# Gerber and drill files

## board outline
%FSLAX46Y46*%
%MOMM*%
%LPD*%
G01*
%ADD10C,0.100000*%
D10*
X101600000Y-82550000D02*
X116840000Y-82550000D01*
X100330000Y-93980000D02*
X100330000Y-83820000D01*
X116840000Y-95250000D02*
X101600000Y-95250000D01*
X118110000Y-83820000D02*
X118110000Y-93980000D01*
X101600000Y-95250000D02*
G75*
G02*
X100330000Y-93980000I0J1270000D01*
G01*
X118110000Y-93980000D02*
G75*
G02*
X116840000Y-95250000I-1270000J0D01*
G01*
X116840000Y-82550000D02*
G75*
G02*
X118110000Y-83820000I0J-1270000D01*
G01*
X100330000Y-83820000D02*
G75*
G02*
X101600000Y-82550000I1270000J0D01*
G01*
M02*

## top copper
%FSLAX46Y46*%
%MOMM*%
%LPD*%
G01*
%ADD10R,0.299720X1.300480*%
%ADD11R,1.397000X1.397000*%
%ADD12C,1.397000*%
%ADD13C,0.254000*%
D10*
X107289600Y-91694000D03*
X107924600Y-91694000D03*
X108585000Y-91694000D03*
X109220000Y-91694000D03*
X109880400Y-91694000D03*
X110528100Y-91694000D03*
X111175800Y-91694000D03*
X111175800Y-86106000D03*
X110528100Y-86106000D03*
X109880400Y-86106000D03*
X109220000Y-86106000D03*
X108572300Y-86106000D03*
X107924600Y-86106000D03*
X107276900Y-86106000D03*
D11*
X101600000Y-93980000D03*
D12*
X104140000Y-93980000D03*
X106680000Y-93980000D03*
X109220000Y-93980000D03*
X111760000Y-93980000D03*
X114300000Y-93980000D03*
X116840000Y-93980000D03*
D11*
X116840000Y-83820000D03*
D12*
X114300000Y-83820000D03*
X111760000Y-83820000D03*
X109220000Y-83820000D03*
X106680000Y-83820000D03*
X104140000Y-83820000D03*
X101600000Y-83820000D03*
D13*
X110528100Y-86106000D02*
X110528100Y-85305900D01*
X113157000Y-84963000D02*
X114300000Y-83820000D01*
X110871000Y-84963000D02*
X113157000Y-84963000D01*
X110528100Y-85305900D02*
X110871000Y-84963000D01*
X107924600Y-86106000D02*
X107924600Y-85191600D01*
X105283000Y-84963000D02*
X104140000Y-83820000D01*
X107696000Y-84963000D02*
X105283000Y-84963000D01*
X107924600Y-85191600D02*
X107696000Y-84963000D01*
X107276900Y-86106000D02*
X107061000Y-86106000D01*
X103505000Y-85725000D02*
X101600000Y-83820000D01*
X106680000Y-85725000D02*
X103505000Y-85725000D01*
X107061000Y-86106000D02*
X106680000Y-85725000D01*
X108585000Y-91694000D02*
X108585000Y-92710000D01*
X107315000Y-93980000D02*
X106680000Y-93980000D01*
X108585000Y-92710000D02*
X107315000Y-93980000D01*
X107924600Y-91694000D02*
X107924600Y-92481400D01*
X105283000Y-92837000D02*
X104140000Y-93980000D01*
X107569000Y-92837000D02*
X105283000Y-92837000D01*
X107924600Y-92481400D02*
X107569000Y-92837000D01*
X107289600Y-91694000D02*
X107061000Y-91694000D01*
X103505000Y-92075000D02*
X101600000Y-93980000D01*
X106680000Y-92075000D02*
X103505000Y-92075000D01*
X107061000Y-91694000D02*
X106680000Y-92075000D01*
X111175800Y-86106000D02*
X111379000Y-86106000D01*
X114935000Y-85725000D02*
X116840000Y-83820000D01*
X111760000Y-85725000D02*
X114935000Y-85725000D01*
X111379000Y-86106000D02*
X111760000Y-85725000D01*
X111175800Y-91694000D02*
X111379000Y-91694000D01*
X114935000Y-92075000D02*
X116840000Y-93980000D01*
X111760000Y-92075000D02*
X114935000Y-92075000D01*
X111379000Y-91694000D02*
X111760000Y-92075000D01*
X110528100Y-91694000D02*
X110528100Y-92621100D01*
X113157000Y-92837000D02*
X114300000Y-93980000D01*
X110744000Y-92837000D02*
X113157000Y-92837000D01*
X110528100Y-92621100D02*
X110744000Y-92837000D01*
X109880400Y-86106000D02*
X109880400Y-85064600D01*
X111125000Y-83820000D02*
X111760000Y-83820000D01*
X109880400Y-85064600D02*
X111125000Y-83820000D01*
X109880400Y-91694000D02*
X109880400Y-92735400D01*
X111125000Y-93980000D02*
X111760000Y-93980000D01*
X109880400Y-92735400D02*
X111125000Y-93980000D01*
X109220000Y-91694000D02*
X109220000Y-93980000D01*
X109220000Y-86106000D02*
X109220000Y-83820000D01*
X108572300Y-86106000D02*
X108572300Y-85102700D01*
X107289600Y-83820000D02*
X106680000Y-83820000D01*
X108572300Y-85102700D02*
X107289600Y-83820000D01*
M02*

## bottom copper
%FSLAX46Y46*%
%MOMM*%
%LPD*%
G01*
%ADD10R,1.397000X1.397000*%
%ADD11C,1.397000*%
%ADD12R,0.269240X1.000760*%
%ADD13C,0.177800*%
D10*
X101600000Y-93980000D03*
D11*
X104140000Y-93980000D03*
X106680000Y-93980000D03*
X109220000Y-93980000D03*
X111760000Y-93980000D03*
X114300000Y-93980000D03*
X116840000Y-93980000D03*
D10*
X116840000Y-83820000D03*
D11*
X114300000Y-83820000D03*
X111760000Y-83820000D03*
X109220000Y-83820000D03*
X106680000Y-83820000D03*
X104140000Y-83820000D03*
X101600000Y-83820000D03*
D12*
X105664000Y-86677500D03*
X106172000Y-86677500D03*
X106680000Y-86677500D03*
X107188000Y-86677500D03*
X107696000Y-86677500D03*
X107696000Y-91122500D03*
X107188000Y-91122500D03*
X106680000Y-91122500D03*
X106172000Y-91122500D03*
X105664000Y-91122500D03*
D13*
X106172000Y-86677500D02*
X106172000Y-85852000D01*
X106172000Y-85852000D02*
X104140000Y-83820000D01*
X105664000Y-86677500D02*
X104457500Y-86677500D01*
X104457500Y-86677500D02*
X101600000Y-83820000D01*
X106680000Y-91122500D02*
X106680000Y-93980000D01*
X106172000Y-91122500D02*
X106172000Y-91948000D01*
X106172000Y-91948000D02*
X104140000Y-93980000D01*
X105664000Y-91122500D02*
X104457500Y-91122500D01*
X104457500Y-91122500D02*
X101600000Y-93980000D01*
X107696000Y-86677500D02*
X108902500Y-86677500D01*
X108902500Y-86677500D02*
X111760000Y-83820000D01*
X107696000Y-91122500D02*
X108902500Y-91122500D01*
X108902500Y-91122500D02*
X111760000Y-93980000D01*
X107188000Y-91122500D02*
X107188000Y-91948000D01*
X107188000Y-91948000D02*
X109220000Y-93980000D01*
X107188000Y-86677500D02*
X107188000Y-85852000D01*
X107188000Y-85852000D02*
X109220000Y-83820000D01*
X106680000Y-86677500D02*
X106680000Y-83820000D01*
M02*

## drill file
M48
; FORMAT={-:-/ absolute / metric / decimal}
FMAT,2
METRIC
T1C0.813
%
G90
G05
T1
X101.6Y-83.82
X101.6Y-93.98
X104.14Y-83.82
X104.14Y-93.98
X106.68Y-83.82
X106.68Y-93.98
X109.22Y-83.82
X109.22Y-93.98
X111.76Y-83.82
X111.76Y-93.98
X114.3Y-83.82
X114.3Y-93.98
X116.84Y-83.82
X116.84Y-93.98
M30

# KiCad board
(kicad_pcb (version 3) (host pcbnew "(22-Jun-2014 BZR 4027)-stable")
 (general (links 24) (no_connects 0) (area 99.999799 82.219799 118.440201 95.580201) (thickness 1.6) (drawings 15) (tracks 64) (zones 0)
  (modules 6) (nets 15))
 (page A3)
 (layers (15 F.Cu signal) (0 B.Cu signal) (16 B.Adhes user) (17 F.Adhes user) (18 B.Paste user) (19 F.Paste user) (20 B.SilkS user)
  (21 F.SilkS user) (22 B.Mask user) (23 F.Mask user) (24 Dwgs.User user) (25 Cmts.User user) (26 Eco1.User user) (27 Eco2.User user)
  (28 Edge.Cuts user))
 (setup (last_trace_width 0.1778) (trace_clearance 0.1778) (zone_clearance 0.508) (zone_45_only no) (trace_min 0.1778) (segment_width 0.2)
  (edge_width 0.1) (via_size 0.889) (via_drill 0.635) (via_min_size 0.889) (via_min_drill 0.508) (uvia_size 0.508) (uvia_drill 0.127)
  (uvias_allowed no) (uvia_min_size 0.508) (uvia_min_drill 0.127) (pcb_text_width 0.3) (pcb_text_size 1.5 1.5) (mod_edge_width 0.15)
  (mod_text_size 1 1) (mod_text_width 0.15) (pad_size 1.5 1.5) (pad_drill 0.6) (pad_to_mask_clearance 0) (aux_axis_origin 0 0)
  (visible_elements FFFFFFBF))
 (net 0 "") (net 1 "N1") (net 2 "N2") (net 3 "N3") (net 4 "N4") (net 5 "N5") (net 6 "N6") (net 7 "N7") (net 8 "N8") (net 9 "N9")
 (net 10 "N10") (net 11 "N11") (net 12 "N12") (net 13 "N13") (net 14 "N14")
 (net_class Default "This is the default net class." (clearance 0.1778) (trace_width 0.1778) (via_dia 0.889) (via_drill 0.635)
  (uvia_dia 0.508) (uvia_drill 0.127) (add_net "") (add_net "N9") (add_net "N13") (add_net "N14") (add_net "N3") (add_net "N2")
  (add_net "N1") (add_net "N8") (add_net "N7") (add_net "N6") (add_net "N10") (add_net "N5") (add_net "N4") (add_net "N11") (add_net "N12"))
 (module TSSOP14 (layer F.Cu) (at 109.22 88.9)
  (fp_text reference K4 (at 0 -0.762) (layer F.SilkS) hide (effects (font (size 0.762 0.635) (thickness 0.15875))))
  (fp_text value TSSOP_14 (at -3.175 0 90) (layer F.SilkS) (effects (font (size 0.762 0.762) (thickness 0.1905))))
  (pad 1 smd rect (at -1.9304 2.794) (size 0.29972 1.30048) (layers F.Cu F.Paste F.Mask) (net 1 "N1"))
  (pad 2 smd rect (at -1.2954 2.794) (size 0.29972 1.30048) (layers F.Cu F.Paste F.Mask) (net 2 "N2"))
  (pad 3 smd rect (at -0.635 2.794) (size 0.29972 1.30048) (layers F.Cu F.Paste F.Mask) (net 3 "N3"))
  (pad 4 smd rect (at 0 2.794) (size 0.29972 1.30048) (layers F.Cu F.Paste F.Mask) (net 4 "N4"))
  (pad 5 smd rect (at 0.6604 2.794) (size 0.29972 1.30048) (layers F.Cu F.Paste F.Mask) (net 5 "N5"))
  (pad 6 smd rect (at 1.3081 2.794) (size 0.29972 1.30048) (layers F.Cu F.Paste F.Mask) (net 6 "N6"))
  (pad 7 smd rect (at 1.9558 2.794) (size 0.29972 1.30048) (layers F.Cu F.Paste F.Mask) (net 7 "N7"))
  (pad 8 smd rect (at 1.9558 -2.794) (size 0.29972 1.30048) (layers F.Cu F.Paste F.Mask) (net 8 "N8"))
  (pad 9 smd rect (at 1.3081 -2.794) (size 0.29972 1.30048) (layers F.Cu F.Paste F.Mask) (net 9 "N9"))
  (pad 10 smd rect (at 0.6604 -2.794) (size 0.29972 1.30048) (layers F.Cu F.Paste F.Mask) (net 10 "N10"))
  (pad 11 smd rect (at 0 -2.794) (size 0.29972 1.30048) (layers F.Cu F.Paste F.Mask) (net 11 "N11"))
  (pad 12 smd rect (at -0.6477 -2.794) (size 0.29972 1.30048) (layers F.Cu F.Paste F.Mask) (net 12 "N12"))
  (pad 13 smd rect (at -1.2954 -2.794) (size 0.29972 1.30048) (layers F.Cu F.Paste F.Mask) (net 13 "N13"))
  (pad 14 smd rect (at -1.9431 -2.794) (size 0.29972 1.30048) (layers F.Cu F.Paste F.Mask) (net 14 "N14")))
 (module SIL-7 (layer F.Cu) (at 109.22 93.98)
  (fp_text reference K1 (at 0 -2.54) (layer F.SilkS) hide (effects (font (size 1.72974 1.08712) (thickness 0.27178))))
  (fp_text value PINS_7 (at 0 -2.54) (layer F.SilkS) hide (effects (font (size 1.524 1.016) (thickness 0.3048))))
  (pad 1 thru_hole rect (at -7.62 0) (size 1.397 1.397) (drill 0.8128) (layers *.Cu *.Mask F.SilkS) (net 1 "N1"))
  (pad 2 thru_hole circle (at -5.08 0) (size 1.397 1.397) (drill 0.8128) (layers *.Cu *.SilkS *.Mask) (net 2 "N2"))
  (pad 3 thru_hole circle (at -2.54 0) (size 1.397 1.397) (drill 0.8128) (layers *.Cu *.SilkS *.Mask) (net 3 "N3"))
  (pad 4 thru_hole circle (at 0 0) (size 1.397 1.397) (drill 0.8128) (layers *.Cu *.SilkS *.Mask) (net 4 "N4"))
  (pad 5 thru_hole circle (at 2.54 0) (size 1.397 1.397) (drill 0.8128) (layers *.Cu *.SilkS *.Mask) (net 5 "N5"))
  (pad 6 thru_hole circle (at 5.08 0) (size 1.397 1.397) (drill 0.8128) (layers *.Cu *.SilkS *.Mask) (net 6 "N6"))
  (pad 7 thru_hole circle (at 7.62 0) (size 1.397 1.397) (drill 0.8128) (layers *.Cu *.SilkS *.Mask) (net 7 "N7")))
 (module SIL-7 (layer F.Cu) (at 109.22 83.82 180)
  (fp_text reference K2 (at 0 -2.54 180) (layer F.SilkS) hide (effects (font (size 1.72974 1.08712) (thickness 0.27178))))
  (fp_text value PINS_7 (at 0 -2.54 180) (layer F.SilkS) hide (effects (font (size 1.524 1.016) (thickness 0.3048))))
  (pad 1 thru_hole rect (at -7.62 0 180) (size 1.397 1.397) (drill 0.8128) (layers *.Cu *.Mask F.SilkS) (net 8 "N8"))
  (pad 2 thru_hole circle (at -5.08 0 180) (size 1.397 1.397) (drill 0.8128) (layers *.Cu *.SilkS *.Mask) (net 9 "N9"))
  (pad 3 thru_hole circle (at -2.54 0 180) (size 1.397 1.397) (drill 0.8128) (layers *.Cu *.SilkS *.Mask) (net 10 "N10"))
  (pad 4 thru_hole circle (at 0 0 180) (size 1.397 1.397) (drill 0.8128) (layers *.Cu *.SilkS *.Mask) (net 11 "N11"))
  (pad 5 thru_hole circle (at 2.54 0 180) (size 1.397 1.397) (drill 0.8128) (layers *.Cu *.SilkS *.Mask) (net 12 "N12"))
  (pad 6 thru_hole circle (at 5.08 0 180) (size 1.397 1.397) (drill 0.8128) (layers *.Cu *.SilkS *.Mask) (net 13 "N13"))
  (pad 7 thru_hole circle (at 7.62 0 180) (size 1.397 1.397) (drill 0.8128) (layers *.Cu *.SilkS *.Mask) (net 14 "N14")))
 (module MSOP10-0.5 (layer B.Cu) (at 106.68 88.9)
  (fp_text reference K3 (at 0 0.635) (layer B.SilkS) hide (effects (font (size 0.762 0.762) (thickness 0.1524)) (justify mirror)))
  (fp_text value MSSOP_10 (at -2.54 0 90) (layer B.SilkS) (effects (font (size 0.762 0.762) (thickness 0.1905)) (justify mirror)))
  (pad 1 smd rect (at -1.016 -2.2225) (size 0.26924 1.00076) (layers B.Cu B.Paste B.Mask) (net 14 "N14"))
  (pad 2 smd rect (at -0.508 -2.2225) (size 0.26924 1.00076) (layers B.Cu B.Paste B.Mask) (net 13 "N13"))
  (pad 3 smd rect (at 0 -2.2225) (size 0.26924 1.00076) (layers B.Cu B.Paste B.Mask) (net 12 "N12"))
  (pad 4 smd rect (at 0.508 -2.2225) (size 0.26924 1.00076) (layers B.Cu B.Paste B.Mask) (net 11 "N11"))
  (pad 5 smd rect (at 1.016 -2.2225) (size 0.26924 1.00076) (layers B.Cu B.Paste B.Mask) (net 10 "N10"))
  (pad 6 smd rect (at 1.016 2.2225) (size 0.26924 1.00076) (layers B.Cu B.Paste B.Mask) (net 5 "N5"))
  (pad 7 smd rect (at 0.508 2.2225) (size 0.26924 1.00076) (layers B.Cu B.Paste B.Mask) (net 4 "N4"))
  (pad 8 smd rect (at 0 2.2225) (size 0.26924 1.00076) (layers B.Cu B.Paste B.Mask) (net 3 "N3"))
  (pad 9 smd rect (at -0.508 2.2225) (size 0.26924 1.00076) (layers B.Cu B.Paste B.Mask) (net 2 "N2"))
  (pad 10 smd rect (at -1.016 2.2225) (size 0.26924 1.00076) (layers B.Cu B.Paste B.Mask) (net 1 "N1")))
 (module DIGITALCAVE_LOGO (layer F.Cu) (at 114.935 88.9 90)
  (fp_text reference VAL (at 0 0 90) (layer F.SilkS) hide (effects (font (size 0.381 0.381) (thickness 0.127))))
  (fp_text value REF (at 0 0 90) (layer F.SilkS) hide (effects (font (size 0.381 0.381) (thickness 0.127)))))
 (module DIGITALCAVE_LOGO (layer B.Cu) (at 114.935 88.9 90)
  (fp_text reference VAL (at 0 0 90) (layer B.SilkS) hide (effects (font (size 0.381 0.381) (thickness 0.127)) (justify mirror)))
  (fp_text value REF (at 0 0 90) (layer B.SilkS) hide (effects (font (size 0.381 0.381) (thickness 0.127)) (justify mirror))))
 (gr_line (start 101.6 82.55) (end 116.84 82.55) (angle 90) (layer Edge.Cuts) (width 0.1))
 (gr_line (start 100.33 93.98) (end 100.33 83.82) (angle 90) (layer Edge.Cuts) (width 0.1))
 (gr_line (start 116.84 95.25) (end 101.6 95.25) (angle 90) (layer Edge.Cuts) (width 0.1))
 (gr_line (start 118.11 83.82) (end 118.11 93.98) (angle 90) (layer Edge.Cuts) (width 0.1))
 (gr_arc (start 101.6 93.98) (end 101.6 95.25) (angle 90) (layer Edge.Cuts) (width 0.1))
 (gr_arc (start 116.84 93.98) (end 118.11 93.98) (angle 90) (layer Edge.Cuts) (width 0.1))
 (gr_arc (start 116.84 83.82) (end 116.84 82.55) (angle 90) (layer Edge.Cuts) (width 0.1))
 (gr_arc (start 101.6 83.82) (end 100.33 83.82) (angle 90) (layer Edge.Cuts) (width 0.1))
 (segment (start 110.5281 86.106) (end 110.5281 85.3059) (width 0.254) (layer F.Cu) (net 9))
 (segment (start 113.157 84.963) (end 114.3 83.82) (width 0.254) (layer F.Cu) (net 9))
 (segment (start 110.871 84.963) (end 113.157 84.963) (width 0.254) (layer F.Cu) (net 9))
 (segment (start 110.5281 85.3059) (end 110.871 84.963) (width 0.254) (layer F.Cu) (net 9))
 (segment (start 106.172 86.6775) (end 106.172 85.852) (width 0.1778) (layer B.Cu) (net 13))
 (segment (start 106.172 85.852) (end 104.14 83.82) (width 0.1778) (layer B.Cu) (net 13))
 (segment (start 107.9246 86.106) (end 107.9246 85.1916) (width 0.254) (layer F.Cu) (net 13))
 (segment (start 105.283 84.963) (end 104.14 83.82) (width 0.254) (layer F.Cu) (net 13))
 (segment (start 107.696 84.963) (end 105.283 84.963) (width 0.254) (layer F.Cu) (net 13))
 (segment (start 107.9246 85.1916) (end 107.696 84.963) (width 0.254) (layer F.Cu) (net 13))
 (segment (start 105.664 86.6775) (end 104.4575 86.6775) (width 0.1778) (layer B.Cu) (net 14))
 (segment (start 104.4575 86.6775) (end 101.6 83.82) (width 0.1778) (layer B.Cu) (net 14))
 (segment (start 107.2769 86.106) (end 107.061 86.106) (width 0.254) (layer F.Cu) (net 14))
 (segment (start 103.505 85.725) (end 101.6 83.82) (width 0.254) (layer F.Cu) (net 14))
 (segment (start 106.68 85.725) (end 103.505 85.725) (width 0.254) (layer F.Cu) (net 14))
 (segment (start 107.061 86.106) (end 106.68 85.725) (width 0.254) (layer F.Cu) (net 14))
 (segment (start 106.68 91.1225) (end 106.68 93.98) (width 0.1778) (layer B.Cu) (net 3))
 (segment (start 108.585 91.694) (end 108.585 92.71) (width 0.254) (layer F.Cu) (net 3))
 (segment (start 107.315 93.98) (end 106.68 93.98) (width 0.254) (layer F.Cu) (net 3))
 (segment (start 108.585 92.71) (end 107.315 93.98) (width 0.254) (layer F.Cu) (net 3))
 (segment (start 106.172 91.1225) (end 106.172 91.948) (width 0.1778) (layer B.Cu) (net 2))
 (segment (start 106.172 91.948) (end 104.14 93.98) (width 0.1778) (layer B.Cu) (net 2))
 (segment (start 107.9246 91.694) (end 107.9246 92.4814) (width 0.254) (layer F.Cu) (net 2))
 (segment (start 105.283 92.837) (end 104.14 93.98) (width 0.254) (layer F.Cu) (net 2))
 (segment (start 107.569 92.837) (end 105.283 92.837) (width 0.254) (layer F.Cu) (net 2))
 (segment (start 107.9246 92.4814) (end 107.569 92.837) (width 0.254) (layer F.Cu) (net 2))
 (segment (start 105.664 91.1225) (end 104.4575 91.1225) (width 0.1778) (layer B.Cu) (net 1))
 (segment (start 104.4575 91.1225) (end 101.6 93.98) (width 0.1778) (layer B.Cu) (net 1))
 (segment (start 107.2896 91.694) (end 107.061 91.694) (width 0.254) (layer F.Cu) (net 1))
 (segment (start 103.505 92.075) (end 101.6 93.98) (width 0.254) (layer F.Cu) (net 1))
 (segment (start 106.68 92.075) (end 103.505 92.075) (width 0.254) (layer F.Cu) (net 1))
 (segment (start 107.061 91.694) (end 106.68 92.075) (width 0.254) (layer F.Cu) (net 1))
 (segment (start 111.1758 86.106) (end 111.379 86.106) (width 0.254) (layer F.Cu) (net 8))
 (segment (start 114.935 85.725) (end 116.84 83.82) (width 0.254) (layer F.Cu) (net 8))
 (segment (start 111.76 85.725) (end 114.935 85.725) (width 0.254) (layer F.Cu) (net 8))
 (segment (start 111.379 86.106) (end 111.76 85.725) (width 0.254) (layer F.Cu) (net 8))
 (segment (start 111.1758 91.694) (end 111.379 91.694) (width 0.254) (layer F.Cu) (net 7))
 (segment (start 114.935 92.075) (end 116.84 93.98) (width 0.254) (layer F.Cu) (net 7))
 (segment (start 111.76 92.075) (end 114.935 92.075) (width 0.254) (layer F.Cu) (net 7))
 (segment (start 111.379 91.694) (end 111.76 92.075) (width 0.254) (layer F.Cu) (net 7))
 (segment (start 110.5281 91.694) (end 110.5281 92.6211) (width 0.254) (layer F.Cu) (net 6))
 (segment (start 113.157 92.837) (end 114.3 93.98) (width 0.254) (layer F.Cu) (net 6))
 (segment (start 110.744 92.837) (end 113.157 92.837) (width 0.254) (layer F.Cu) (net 6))
 (segment (start 110.5281 92.6211) (end 110.744 92.837) (width 0.254) (layer F.Cu) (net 6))
 (segment (start 107.696 86.6775) (end 108.9025 86.6775) (width 0.1778) (layer B.Cu) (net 10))
 (segment (start 108.9025 86.6775) (end 111.76 83.82) (width 0.1778) (layer B.Cu) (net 10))
 (segment (start 109.8804 86.106) (end 109.8804 85.0646) (width 0.254) (layer F.Cu) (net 10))
 (segment (start 111.125 83.82) (end 111.76 83.82) (width 0.254) (layer F.Cu) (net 10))
 (segment (start 109.8804 85.0646) (end 111.125 83.82) (width 0.254) (layer F.Cu) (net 10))
 (segment (start 107.696 91.1225) (end 108.9025 91.1225) (width 0.1778) (layer B.Cu) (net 5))
 (segment (start 108.9025 91.1225) (end 111.76 93.98) (width 0.1778) (layer B.Cu) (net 5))
 (segment (start 109.8804 91.694) (end 109.8804 92.7354) (width 0.254) (layer F.Cu) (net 5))
 (segment (start 111.125 93.98) (end 111.76 93.98) (width 0.254) (layer F.Cu) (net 5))
 (segment (start 109.8804 92.7354) (end 111.125 93.98) (width 0.254) (layer F.Cu) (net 5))
 (segment (start 107.188 91.1225) (end 107.188 91.948) (width 0.1778) (layer B.Cu) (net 4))
 (segment (start 107.188 91.948) (end 109.22 93.98) (width 0.1778) (layer B.Cu) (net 4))
 (segment (start 109.22 91.694) (end 109.22 93.98) (width 0.254) (layer F.Cu) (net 4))
 (segment (start 107.188 86.6775) (end 107.188 85.852) (width 0.1778) (layer B.Cu) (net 11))
 (segment (start 107.188 85.852) (end 109.22 83.82) (width 0.1778) (layer B.Cu) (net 11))
 (segment (start 109.22 86.106) (end 109.22 83.82) (width 0.254) (layer F.Cu) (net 11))
 (segment (start 106.68 86.6775) (end 106.68 83.82) (width 0.1778) (layer B.Cu) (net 12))
 (segment (start 108.5723 86.106) (end 108.5723 85.1027) (width 0.254) (layer F.Cu) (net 12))
 (segment (start 107.2896 83.82) (end 106.68 83.82) (width 0.254) (layer F.Cu) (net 12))
 (segment (start 108.5723 85.1027) (end 107.2896 83.82) (width 0.254) (layer F.Cu) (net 12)))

